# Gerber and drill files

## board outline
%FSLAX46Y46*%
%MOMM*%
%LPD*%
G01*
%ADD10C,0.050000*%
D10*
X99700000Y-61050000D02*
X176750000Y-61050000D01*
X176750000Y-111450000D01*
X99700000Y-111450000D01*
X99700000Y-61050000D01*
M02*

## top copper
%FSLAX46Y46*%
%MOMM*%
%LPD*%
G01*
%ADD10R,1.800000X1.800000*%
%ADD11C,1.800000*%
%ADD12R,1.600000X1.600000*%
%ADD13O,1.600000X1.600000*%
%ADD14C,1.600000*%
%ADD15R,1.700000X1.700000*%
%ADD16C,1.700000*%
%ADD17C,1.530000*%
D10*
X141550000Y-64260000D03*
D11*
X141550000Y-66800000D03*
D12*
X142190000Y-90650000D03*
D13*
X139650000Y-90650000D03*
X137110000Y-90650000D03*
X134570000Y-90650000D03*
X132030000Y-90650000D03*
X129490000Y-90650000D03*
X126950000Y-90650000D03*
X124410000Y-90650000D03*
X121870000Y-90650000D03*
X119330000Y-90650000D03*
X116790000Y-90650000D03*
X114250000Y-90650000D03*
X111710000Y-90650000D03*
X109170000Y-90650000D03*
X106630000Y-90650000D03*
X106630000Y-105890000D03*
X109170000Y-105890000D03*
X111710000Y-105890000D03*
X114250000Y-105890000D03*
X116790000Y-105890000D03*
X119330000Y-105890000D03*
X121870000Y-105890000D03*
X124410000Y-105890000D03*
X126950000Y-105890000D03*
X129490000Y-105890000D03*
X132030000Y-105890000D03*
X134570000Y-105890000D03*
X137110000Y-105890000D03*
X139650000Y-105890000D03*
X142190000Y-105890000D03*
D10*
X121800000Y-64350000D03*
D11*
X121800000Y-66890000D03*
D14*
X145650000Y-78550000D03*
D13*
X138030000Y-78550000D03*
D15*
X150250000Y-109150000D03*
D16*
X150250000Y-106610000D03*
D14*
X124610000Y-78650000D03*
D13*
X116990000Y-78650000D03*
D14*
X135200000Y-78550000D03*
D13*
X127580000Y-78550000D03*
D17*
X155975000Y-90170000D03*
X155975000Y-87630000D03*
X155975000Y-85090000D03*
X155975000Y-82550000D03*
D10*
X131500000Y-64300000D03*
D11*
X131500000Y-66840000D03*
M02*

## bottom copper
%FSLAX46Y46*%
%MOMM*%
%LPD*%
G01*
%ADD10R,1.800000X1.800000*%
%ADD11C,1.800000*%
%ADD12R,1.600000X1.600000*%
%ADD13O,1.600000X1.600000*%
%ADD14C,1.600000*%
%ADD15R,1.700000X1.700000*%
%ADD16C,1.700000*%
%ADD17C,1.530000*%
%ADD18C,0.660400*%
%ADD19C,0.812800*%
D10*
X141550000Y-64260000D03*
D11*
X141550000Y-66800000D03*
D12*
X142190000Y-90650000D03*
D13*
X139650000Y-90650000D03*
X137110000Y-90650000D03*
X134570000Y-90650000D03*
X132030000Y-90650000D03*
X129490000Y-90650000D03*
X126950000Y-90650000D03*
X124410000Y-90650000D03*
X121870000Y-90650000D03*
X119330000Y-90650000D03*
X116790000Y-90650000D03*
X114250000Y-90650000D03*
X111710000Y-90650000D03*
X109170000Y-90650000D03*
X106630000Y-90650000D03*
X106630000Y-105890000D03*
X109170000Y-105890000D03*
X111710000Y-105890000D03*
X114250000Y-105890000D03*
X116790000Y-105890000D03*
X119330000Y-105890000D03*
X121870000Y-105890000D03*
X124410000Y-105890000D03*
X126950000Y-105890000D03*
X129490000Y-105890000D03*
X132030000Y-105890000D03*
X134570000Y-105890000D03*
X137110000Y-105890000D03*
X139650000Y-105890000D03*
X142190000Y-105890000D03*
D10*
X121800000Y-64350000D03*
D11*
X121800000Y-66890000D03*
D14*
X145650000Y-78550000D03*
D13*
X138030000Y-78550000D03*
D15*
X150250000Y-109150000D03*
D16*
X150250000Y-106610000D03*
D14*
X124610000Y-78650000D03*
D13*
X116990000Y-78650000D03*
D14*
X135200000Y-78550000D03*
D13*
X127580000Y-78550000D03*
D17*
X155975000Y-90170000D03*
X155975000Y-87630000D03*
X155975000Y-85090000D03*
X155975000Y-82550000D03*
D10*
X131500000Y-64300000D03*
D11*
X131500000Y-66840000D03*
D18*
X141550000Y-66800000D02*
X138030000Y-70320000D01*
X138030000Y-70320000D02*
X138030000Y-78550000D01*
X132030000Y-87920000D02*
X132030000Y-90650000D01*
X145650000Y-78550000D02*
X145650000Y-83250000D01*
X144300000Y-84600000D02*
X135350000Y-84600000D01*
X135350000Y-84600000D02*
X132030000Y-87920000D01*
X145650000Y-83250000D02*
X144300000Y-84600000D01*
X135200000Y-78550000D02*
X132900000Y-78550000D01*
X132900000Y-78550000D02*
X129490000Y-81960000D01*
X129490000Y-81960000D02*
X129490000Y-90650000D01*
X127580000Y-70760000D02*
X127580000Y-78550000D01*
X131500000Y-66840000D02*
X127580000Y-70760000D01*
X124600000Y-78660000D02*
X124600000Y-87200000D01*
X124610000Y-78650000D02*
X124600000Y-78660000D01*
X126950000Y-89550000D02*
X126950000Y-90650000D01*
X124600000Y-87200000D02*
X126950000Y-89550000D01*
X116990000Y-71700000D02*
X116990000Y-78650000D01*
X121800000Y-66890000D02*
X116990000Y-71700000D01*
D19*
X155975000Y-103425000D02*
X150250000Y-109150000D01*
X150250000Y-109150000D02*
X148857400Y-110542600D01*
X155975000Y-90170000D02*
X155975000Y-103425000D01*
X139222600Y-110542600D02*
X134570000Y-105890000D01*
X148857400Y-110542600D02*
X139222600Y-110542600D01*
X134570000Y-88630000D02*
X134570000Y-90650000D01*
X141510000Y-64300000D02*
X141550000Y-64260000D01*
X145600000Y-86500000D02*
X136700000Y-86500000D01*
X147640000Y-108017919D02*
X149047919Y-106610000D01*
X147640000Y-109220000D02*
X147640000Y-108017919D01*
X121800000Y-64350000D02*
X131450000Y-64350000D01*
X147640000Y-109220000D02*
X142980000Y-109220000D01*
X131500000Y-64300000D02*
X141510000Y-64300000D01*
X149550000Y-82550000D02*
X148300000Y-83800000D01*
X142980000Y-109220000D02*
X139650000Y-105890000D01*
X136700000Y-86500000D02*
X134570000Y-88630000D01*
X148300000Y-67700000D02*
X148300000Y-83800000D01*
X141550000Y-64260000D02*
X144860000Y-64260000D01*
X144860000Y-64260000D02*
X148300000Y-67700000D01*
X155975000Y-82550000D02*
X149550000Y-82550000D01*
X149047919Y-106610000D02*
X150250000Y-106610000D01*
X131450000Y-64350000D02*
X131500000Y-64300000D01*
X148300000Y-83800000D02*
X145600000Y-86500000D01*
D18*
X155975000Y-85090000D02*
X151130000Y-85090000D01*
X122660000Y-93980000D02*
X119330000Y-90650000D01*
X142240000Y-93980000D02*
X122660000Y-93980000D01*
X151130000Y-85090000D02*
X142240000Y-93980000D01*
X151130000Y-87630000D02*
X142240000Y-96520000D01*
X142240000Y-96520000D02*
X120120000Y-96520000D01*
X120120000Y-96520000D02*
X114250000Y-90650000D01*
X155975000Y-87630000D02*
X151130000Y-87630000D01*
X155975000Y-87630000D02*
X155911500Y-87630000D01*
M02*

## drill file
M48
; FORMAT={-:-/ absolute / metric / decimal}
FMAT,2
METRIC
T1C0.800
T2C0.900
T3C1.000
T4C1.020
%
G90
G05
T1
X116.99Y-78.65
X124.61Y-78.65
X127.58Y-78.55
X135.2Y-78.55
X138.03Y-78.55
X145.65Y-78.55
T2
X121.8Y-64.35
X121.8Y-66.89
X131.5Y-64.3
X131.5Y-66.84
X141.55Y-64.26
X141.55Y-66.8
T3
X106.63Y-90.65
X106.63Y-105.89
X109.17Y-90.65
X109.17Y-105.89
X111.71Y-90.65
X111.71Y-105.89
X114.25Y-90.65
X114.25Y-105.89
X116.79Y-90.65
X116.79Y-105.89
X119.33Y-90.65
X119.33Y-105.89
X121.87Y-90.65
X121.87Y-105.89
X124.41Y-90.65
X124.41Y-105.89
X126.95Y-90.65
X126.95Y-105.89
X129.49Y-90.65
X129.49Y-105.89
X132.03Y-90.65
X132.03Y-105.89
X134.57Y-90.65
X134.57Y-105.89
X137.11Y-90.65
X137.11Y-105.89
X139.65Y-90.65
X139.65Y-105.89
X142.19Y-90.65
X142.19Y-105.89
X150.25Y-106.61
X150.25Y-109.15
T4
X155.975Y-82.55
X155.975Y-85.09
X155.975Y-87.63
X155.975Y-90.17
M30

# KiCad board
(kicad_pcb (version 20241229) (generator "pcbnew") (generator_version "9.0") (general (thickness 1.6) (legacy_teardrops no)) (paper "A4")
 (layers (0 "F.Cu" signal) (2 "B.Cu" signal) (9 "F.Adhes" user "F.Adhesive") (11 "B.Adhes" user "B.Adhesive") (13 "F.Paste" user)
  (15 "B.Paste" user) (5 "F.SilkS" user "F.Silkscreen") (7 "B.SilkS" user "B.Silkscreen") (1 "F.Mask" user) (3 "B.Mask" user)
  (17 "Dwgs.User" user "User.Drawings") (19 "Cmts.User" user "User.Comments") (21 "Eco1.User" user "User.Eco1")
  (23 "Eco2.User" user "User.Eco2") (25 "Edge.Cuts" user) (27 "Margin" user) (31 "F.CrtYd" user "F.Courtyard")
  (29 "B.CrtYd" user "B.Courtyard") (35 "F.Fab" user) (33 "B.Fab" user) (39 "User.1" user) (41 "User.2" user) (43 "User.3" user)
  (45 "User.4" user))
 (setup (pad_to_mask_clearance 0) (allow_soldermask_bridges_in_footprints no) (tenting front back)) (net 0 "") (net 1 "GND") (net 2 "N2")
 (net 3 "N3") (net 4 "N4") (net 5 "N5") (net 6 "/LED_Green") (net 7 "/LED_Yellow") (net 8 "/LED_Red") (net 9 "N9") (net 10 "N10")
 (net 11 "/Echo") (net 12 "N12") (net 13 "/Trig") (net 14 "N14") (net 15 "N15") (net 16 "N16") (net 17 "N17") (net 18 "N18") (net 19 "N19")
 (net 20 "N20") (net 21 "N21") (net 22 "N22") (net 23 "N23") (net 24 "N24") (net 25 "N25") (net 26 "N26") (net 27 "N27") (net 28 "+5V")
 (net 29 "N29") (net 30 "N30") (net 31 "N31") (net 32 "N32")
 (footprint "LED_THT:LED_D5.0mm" (layer "F.Cu") (at 141.55 64.26 -90)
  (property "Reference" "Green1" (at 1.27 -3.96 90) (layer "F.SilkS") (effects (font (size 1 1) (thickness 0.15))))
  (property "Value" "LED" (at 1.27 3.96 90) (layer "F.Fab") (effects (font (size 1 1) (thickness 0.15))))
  (pad "1" thru_hole rect (at 0 0 270) (size 1.8 1.8) (drill 0.9) (layers "*.Cu" "*.Mask") (remove_unused_layers no) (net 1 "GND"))
  (pad "2" thru_hole circle (at 2.54 0 270) (size 1.8 1.8) (drill 0.9) (layers "*.Cu" "*.Mask") (remove_unused_layers no) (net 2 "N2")))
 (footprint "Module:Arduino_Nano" (layer "F.Cu") (at 142.19 90.65 -90)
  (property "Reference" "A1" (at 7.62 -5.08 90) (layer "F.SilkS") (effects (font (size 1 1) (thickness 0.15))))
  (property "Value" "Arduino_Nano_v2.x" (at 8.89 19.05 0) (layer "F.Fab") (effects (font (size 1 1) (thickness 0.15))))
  (pad "1" thru_hole rect (at 0 0 270) (size 1.6 1.6) (drill 1) (layers "*.Cu" "*.Mask") (remove_unused_layers no) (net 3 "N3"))
  (pad "2" thru_hole oval (at 0 2.54 270) (size 1.6 1.6) (drill 1) (layers "*.Cu" "*.Mask") (remove_unused_layers no) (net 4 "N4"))
  (pad "3" thru_hole oval (at 0 5.08 270) (size 1.6 1.6) (drill 1) (layers "*.Cu" "*.Mask") (remove_unused_layers no) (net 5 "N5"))
  (pad "4" thru_hole oval (at 0 7.62 270) (size 1.6 1.6) (drill 1) (layers "*.Cu" "*.Mask") (remove_unused_layers no) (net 1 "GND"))
  (pad "5" thru_hole oval (at 0 10.16 270) (size 1.6 1.6) (drill 1) (layers "*.Cu" "*.Mask") (remove_unused_layers no) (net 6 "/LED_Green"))
  (pad "6" thru_hole oval (at 0 12.7 270) (size 1.6 1.6) (drill 1) (layers "*.Cu" "*.Mask") (remove_unused_layers no) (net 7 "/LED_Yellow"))
  (pad "7" thru_hole oval (at 0 15.24 270) (size 1.6 1.6) (drill 1) (layers "*.Cu" "*.Mask") (remove_unused_layers no) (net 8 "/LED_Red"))
  (pad "8" thru_hole oval (at 0 17.78 270) (size 1.6 1.6) (drill 1) (layers "*.Cu" "*.Mask") (remove_unused_layers no) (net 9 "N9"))
  (pad "9" thru_hole oval (at 0 20.32 270) (size 1.6 1.6) (drill 1) (layers "*.Cu" "*.Mask") (remove_unused_layers no) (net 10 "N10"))
  (pad "10" thru_hole oval (at 0 22.86 270) (size 1.6 1.6) (drill 1) (layers "*.Cu" "*.Mask") (remove_unused_layers no) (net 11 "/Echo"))
  (pad "11" thru_hole oval (at 0 25.4 270) (size 1.6 1.6) (drill 1) (layers "*.Cu" "*.Mask") (remove_unused_layers no) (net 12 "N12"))
  (pad "12" thru_hole oval (at 0 27.94 270) (size 1.6 1.6) (drill 1) (layers "*.Cu" "*.Mask") (remove_unused_layers no) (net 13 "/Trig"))
  (pad "13" thru_hole oval (at 0 30.48 270) (size 1.6 1.6) (drill 1) (layers "*.Cu" "*.Mask") (remove_unused_layers no) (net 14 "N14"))
  (pad "14" thru_hole oval (at 0 33.02 270) (size 1.6 1.6) (drill 1) (layers "*.Cu" "*.Mask") (remove_unused_layers no) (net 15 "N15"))
  (pad "15" thru_hole oval (at 0 35.56 270) (size 1.6 1.6) (drill 1) (layers "*.Cu" "*.Mask") (remove_unused_layers no) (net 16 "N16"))
  (pad "16" thru_hole oval (at 15.24 35.56 270) (size 1.6 1.6) (drill 1) (layers "*.Cu" "*.Mask") (remove_unused_layers no) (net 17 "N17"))
  (pad "17" thru_hole oval (at 15.24 33.02 270) (size 1.6 1.6) (drill 1) (layers "*.Cu" "*.Mask") (remove_unused_layers no) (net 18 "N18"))
  (pad "18" thru_hole oval (at 15.24 30.48 270) (size 1.6 1.6) (drill 1) (layers "*.Cu" "*.Mask") (remove_unused_layers no) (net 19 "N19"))
  (pad "19" thru_hole oval (at 15.24 27.94 270) (size 1.6 1.6) (drill 1) (layers "*.Cu" "*.Mask") (remove_unused_layers no) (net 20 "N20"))
  (pad "20" thru_hole oval (at 15.24 25.4 270) (size 1.6 1.6) (drill 1) (layers "*.Cu" "*.Mask") (remove_unused_layers no) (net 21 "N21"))
  (pad "21" thru_hole oval (at 15.24 22.86 270) (size 1.6 1.6) (drill 1) (layers "*.Cu" "*.Mask") (remove_unused_layers no) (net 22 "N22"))
  (pad "22" thru_hole oval (at 15.24 20.32 270) (size 1.6 1.6) (drill 1) (layers "*.Cu" "*.Mask") (remove_unused_layers no) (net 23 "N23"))
  (pad "23" thru_hole oval (at 15.24 17.78 270) (size 1.6 1.6) (drill 1) (layers "*.Cu" "*.Mask") (remove_unused_layers no) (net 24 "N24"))
  (pad "24" thru_hole oval (at 15.24 15.24 270) (size 1.6 1.6) (drill 1) (layers "*.Cu" "*.Mask") (remove_unused_layers no) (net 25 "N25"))
  (pad "25" thru_hole oval (at 15.24 12.7 270) (size 1.6 1.6) (drill 1) (layers "*.Cu" "*.Mask") (remove_unused_layers no) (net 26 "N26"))
  (pad "26" thru_hole oval (at 15.24 10.16 270) (size 1.6 1.6) (drill 1) (layers "*.Cu" "*.Mask") (remove_unused_layers no) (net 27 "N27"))
  (pad "27" thru_hole oval (at 15.24 7.62 270) (size 1.6 1.6) (drill 1) (layers "*.Cu" "*.Mask") (remove_unused_layers no) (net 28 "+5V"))
  (pad "28" thru_hole oval (at 15.24 5.08 270) (size 1.6 1.6) (drill 1) (layers "*.Cu" "*.Mask") (remove_unused_layers no) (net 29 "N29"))
  (pad "29" thru_hole oval (at 15.24 2.54 270) (size 1.6 1.6) (drill 1) (layers "*.Cu" "*.Mask") (remove_unused_layers no) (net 1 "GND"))
  (pad "30" thru_hole oval (at 15.24 0 270) (size 1.6 1.6) (drill 1) (layers "*.Cu" "*.Mask") (remove_unused_layers no) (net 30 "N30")))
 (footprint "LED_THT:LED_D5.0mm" (layer "F.Cu") (at 121.8 64.35 -90)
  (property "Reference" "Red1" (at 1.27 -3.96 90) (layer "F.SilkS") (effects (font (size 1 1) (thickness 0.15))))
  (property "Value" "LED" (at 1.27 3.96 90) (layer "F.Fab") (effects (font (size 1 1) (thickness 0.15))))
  (pad "1" thru_hole rect (at 0 0 270) (size 1.8 1.8) (drill 0.9) (layers "*.Cu" "*.Mask") (remove_unused_layers no) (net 1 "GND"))
  (pad "2" thru_hole circle (at 2.54 0 270) (size 1.8 1.8) (drill 0.9) (layers "*.Cu" "*.Mask") (remove_unused_layers no) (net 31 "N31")))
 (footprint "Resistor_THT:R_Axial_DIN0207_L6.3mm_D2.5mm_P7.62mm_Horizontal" (layer "F.Cu") (at 145.65 78.55 180)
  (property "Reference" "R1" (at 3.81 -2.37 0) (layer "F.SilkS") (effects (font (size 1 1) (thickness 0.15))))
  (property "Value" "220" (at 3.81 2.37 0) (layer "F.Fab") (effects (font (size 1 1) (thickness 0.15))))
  (pad "1" thru_hole circle (at 0 0 180) (size 1.6 1.6) (drill 0.8) (layers "*.Cu" "*.Mask") (remove_unused_layers no) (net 6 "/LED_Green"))
  (pad "2" thru_hole oval (at 7.62 0 180) (size 1.6 1.6) (drill 0.8) (layers "*.Cu" "*.Mask") (remove_unused_layers no) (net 2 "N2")))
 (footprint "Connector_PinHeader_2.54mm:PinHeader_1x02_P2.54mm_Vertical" (layer "F.Cu") (at 150.25 109.15 180)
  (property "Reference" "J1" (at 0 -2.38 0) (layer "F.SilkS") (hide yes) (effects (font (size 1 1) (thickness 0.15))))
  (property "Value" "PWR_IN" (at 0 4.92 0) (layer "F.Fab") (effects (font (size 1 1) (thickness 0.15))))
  (pad "1" thru_hole rect (at 0 0 180) (size 1.7 1.7) (drill 1) (layers "*.Cu" "*.Mask") (remove_unused_layers no) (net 28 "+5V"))
  (pad "2" thru_hole circle (at 0 2.54 180) (size 1.7 1.7) (drill 1) (layers "*.Cu" "*.Mask") (remove_unused_layers no) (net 1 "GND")))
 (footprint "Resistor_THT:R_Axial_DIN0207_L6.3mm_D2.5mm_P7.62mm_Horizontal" (layer "F.Cu") (at 124.61 78.65 180)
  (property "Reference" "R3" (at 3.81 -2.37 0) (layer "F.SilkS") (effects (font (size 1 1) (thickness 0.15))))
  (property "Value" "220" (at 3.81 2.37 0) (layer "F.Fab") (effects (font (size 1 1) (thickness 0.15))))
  (pad "1" thru_hole circle (at 0 0 180) (size 1.6 1.6) (drill 0.8) (layers "*.Cu" "*.Mask") (remove_unused_layers no) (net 8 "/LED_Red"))
  (pad "2" thru_hole oval (at 7.62 0 180) (size 1.6 1.6) (drill 0.8) (layers "*.Cu" "*.Mask") (remove_unused_layers no) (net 31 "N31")))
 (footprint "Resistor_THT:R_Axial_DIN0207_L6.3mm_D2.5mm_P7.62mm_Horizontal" (layer "F.Cu") (at 135.2 78.55 180)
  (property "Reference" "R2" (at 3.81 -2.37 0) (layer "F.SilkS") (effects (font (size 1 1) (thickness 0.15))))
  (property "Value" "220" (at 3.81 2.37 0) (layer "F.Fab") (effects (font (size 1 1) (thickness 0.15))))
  (pad "1" thru_hole circle (at 0 0 180) (size 1.6 1.6) (drill 0.8) (layers "*.Cu" "*.Mask") (remove_unused_layers no) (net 7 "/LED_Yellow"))
  (pad "2" thru_hole oval (at 7.62 0 180) (size 1.6 1.6) (drill 0.8) (layers "*.Cu" "*.Mask") (remove_unused_layers no) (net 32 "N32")))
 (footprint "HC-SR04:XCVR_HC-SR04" (layer "F.Cu") (at 155.975 86.36 90)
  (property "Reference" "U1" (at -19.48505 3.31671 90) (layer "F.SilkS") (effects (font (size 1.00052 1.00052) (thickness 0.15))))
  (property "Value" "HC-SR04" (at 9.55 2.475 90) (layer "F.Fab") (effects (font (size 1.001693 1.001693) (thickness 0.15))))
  (pad "1" thru_hole circle (at -3.81 0 90) (size 1.53 1.53) (drill 1.02) (layers "*.Cu" "*.Mask") (remove_unused_layers no) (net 28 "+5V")
   (solder_mask_margin 0.102))
  (pad "2" thru_hole circle (at -1.27 0 90) (size 1.53 1.53) (drill 1.02) (layers "*.Cu" "*.Mask") (remove_unused_layers no)
   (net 13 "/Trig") (solder_mask_margin 0.102))
  (pad "3" thru_hole circle (at 1.27 0 90) (size 1.53 1.53) (drill 1.02) (layers "*.Cu" "*.Mask") (remove_unused_layers no) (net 11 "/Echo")
   (solder_mask_margin 0.102))
  (pad "4" thru_hole circle (at 3.81 0 90) (size 1.53 1.53) (drill 1.02) (layers "*.Cu" "*.Mask") (remove_unused_layers no) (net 1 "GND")
   (solder_mask_margin 0.102)))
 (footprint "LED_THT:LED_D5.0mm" (layer "F.Cu") (at 131.5 64.3 -90)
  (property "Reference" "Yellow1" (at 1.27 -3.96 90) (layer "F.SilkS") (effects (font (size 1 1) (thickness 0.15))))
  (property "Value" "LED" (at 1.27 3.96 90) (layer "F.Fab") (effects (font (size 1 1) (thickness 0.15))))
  (pad "1" thru_hole rect (at 0 0 270) (size 1.8 1.8) (drill 0.9) (layers "*.Cu" "*.Mask") (remove_unused_layers no) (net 1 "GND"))
  (pad "2" thru_hole circle (at 2.54 0 270) (size 1.8 1.8) (drill 0.9) (layers "*.Cu" "*.Mask") (remove_unused_layers no) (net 32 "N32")))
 (gr_rect (start 99.7 61.05) (end 176.75 111.45) (stroke (width 0.05) (type default)) (fill no) (layer "Edge.Cuts"))
 (segment (start 141.55 66.8) (end 138.03 70.32) (width 0.6604) (layer "B.Cu") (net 2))
 (segment (start 138.03 70.32) (end 138.03 78.55) (width 0.6604) (layer "B.Cu") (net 2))
 (segment (start 132.03 87.92) (end 132.03 90.65) (width 0.6604) (layer "B.Cu") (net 6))
 (segment (start 145.65 78.55) (end 145.65 83.25) (width 0.6604) (layer "B.Cu") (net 6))
 (segment (start 144.3 84.6) (end 135.35 84.6) (width 0.6604) (layer "B.Cu") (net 6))
 (segment (start 135.35 84.6) (end 132.03 87.92) (width 0.6604) (layer "B.Cu") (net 6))
 (segment (start 145.65 83.25) (end 144.3 84.6) (width 0.6604) (layer "B.Cu") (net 6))
 (segment (start 135.2 78.55) (end 132.9 78.55) (width 0.6604) (layer "B.Cu") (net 7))
 (segment (start 132.9 78.55) (end 129.49 81.96) (width 0.6604) (layer "B.Cu") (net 7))
 (segment (start 129.49 81.96) (end 129.49 90.65) (width 0.6604) (layer "B.Cu") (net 7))
 (segment (start 127.58 70.76) (end 127.58 78.55) (width 0.6604) (layer "B.Cu") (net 32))
 (segment (start 131.5 66.84) (end 127.58 70.76) (width 0.6604) (layer "B.Cu") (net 32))
 (segment (start 124.6 78.66) (end 124.6 87.2) (width 0.6604) (layer "B.Cu") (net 8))
 (segment (start 124.61 78.65) (end 124.6 78.66) (width 0.6604) (layer "B.Cu") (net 8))
 (segment (start 126.95 89.55) (end 126.95 90.65) (width 0.6604) (layer "B.Cu") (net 8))
 (segment (start 124.6 87.2) (end 126.95 89.55) (width 0.6604) (layer "B.Cu") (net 8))
 (segment (start 116.99 71.7) (end 116.99 78.65) (width 0.6604) (layer "B.Cu") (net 31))
 (segment (start 121.8 66.89) (end 116.99 71.7) (width 0.6604) (layer "B.Cu") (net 31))
 (segment (start 155.975 103.425) (end 150.25 109.15) (width 0.8128) (layer "B.Cu") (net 28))
 (segment (start 150.25 109.15) (end 148.8574 110.5426) (width 0.8128) (layer "B.Cu") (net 28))
 (segment (start 155.975 90.17) (end 155.975 103.425) (width 0.8128) (layer "B.Cu") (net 28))
 (segment (start 139.2226 110.5426) (end 134.57 105.89) (width 0.8128) (layer "B.Cu") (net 28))
 (segment (start 148.8574 110.5426) (end 139.2226 110.5426) (width 0.8128) (layer "B.Cu") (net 28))
 (segment (start 134.57 88.63) (end 134.57 90.65) (width 0.8128) (layer "B.Cu") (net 1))
 (segment (start 141.51 64.3) (end 141.55 64.26) (width 0.8128) (layer "B.Cu") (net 1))
 (segment (start 145.6 86.5) (end 136.7 86.5) (width 0.8128) (layer "B.Cu") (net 1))
 (segment (start 147.64 108.017919) (end 149.047919 106.61) (width 0.8128) (layer "B.Cu") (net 1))
 (segment (start 147.64 109.22) (end 147.64 108.017919) (width 0.8128) (layer "B.Cu") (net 1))
 (segment (start 121.8 64.35) (end 131.45 64.35) (width 0.8128) (layer "B.Cu") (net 1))
 (segment (start 147.64 109.22) (end 142.98 109.22) (width 0.8128) (layer "B.Cu") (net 1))
 (segment (start 131.5 64.3) (end 141.51 64.3) (width 0.8128) (layer "B.Cu") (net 1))
 (segment (start 149.55 82.55) (end 148.3 83.8) (width 0.8128) (layer "B.Cu") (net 1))
 (segment (start 142.98 109.22) (end 139.65 105.89) (width 0.8128) (layer "B.Cu") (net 1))
 (segment (start 136.7 86.5) (end 134.57 88.63) (width 0.8128) (layer "B.Cu") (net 1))
 (segment (start 148.3 67.7) (end 148.3 83.8) (width 0.8128) (layer "B.Cu") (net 1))
 (segment (start 141.55 64.26) (end 144.86 64.26) (width 0.8128) (layer "B.Cu") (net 1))
 (segment (start 144.86 64.26) (end 148.3 67.7) (width 0.8128) (layer "B.Cu") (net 1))
 (segment (start 155.975 82.55) (end 149.55 82.55) (width 0.8128) (layer "B.Cu") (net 1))
 (segment (start 149.047919 106.61) (end 150.25 106.61) (width 0.8128) (layer "B.Cu") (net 1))
 (segment (start 131.45 64.35) (end 131.5 64.3) (width 0.8128) (layer "B.Cu") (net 1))
 (segment (start 148.3 83.8) (end 145.6 86.5) (width 0.8128) (layer "B.Cu") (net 1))
 (segment (start 155.975 85.09) (end 151.13 85.09) (width 0.6604) (layer "B.Cu") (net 11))
 (segment (start 122.66 93.98) (end 119.33 90.65) (width 0.6604) (layer "B.Cu") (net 11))
 (segment (start 142.24 93.98) (end 122.66 93.98) (width 0.6604) (layer "B.Cu") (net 11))
 (segment (start 151.13 85.09) (end 142.24 93.98) (width 0.6604) (layer "B.Cu") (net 11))
 (segment (start 151.13 87.63) (end 142.24 96.52) (width 0.6604) (layer "B.Cu") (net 13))
 (segment (start 142.24 96.52) (end 120.12 96.52) (width 0.6604) (layer "B.Cu") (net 13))
 (segment (start 120.12 96.52) (end 114.25 90.65) (width 0.6604) (layer "B.Cu") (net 13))
 (segment (start 155.975 87.63) (end 151.13 87.63) (width 0.6604) (layer "B.Cu") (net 13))
 (segment (start 155.975 87.63) (end 155.9115 87.63) (width 0.6604) (layer "B.Cu") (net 13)))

